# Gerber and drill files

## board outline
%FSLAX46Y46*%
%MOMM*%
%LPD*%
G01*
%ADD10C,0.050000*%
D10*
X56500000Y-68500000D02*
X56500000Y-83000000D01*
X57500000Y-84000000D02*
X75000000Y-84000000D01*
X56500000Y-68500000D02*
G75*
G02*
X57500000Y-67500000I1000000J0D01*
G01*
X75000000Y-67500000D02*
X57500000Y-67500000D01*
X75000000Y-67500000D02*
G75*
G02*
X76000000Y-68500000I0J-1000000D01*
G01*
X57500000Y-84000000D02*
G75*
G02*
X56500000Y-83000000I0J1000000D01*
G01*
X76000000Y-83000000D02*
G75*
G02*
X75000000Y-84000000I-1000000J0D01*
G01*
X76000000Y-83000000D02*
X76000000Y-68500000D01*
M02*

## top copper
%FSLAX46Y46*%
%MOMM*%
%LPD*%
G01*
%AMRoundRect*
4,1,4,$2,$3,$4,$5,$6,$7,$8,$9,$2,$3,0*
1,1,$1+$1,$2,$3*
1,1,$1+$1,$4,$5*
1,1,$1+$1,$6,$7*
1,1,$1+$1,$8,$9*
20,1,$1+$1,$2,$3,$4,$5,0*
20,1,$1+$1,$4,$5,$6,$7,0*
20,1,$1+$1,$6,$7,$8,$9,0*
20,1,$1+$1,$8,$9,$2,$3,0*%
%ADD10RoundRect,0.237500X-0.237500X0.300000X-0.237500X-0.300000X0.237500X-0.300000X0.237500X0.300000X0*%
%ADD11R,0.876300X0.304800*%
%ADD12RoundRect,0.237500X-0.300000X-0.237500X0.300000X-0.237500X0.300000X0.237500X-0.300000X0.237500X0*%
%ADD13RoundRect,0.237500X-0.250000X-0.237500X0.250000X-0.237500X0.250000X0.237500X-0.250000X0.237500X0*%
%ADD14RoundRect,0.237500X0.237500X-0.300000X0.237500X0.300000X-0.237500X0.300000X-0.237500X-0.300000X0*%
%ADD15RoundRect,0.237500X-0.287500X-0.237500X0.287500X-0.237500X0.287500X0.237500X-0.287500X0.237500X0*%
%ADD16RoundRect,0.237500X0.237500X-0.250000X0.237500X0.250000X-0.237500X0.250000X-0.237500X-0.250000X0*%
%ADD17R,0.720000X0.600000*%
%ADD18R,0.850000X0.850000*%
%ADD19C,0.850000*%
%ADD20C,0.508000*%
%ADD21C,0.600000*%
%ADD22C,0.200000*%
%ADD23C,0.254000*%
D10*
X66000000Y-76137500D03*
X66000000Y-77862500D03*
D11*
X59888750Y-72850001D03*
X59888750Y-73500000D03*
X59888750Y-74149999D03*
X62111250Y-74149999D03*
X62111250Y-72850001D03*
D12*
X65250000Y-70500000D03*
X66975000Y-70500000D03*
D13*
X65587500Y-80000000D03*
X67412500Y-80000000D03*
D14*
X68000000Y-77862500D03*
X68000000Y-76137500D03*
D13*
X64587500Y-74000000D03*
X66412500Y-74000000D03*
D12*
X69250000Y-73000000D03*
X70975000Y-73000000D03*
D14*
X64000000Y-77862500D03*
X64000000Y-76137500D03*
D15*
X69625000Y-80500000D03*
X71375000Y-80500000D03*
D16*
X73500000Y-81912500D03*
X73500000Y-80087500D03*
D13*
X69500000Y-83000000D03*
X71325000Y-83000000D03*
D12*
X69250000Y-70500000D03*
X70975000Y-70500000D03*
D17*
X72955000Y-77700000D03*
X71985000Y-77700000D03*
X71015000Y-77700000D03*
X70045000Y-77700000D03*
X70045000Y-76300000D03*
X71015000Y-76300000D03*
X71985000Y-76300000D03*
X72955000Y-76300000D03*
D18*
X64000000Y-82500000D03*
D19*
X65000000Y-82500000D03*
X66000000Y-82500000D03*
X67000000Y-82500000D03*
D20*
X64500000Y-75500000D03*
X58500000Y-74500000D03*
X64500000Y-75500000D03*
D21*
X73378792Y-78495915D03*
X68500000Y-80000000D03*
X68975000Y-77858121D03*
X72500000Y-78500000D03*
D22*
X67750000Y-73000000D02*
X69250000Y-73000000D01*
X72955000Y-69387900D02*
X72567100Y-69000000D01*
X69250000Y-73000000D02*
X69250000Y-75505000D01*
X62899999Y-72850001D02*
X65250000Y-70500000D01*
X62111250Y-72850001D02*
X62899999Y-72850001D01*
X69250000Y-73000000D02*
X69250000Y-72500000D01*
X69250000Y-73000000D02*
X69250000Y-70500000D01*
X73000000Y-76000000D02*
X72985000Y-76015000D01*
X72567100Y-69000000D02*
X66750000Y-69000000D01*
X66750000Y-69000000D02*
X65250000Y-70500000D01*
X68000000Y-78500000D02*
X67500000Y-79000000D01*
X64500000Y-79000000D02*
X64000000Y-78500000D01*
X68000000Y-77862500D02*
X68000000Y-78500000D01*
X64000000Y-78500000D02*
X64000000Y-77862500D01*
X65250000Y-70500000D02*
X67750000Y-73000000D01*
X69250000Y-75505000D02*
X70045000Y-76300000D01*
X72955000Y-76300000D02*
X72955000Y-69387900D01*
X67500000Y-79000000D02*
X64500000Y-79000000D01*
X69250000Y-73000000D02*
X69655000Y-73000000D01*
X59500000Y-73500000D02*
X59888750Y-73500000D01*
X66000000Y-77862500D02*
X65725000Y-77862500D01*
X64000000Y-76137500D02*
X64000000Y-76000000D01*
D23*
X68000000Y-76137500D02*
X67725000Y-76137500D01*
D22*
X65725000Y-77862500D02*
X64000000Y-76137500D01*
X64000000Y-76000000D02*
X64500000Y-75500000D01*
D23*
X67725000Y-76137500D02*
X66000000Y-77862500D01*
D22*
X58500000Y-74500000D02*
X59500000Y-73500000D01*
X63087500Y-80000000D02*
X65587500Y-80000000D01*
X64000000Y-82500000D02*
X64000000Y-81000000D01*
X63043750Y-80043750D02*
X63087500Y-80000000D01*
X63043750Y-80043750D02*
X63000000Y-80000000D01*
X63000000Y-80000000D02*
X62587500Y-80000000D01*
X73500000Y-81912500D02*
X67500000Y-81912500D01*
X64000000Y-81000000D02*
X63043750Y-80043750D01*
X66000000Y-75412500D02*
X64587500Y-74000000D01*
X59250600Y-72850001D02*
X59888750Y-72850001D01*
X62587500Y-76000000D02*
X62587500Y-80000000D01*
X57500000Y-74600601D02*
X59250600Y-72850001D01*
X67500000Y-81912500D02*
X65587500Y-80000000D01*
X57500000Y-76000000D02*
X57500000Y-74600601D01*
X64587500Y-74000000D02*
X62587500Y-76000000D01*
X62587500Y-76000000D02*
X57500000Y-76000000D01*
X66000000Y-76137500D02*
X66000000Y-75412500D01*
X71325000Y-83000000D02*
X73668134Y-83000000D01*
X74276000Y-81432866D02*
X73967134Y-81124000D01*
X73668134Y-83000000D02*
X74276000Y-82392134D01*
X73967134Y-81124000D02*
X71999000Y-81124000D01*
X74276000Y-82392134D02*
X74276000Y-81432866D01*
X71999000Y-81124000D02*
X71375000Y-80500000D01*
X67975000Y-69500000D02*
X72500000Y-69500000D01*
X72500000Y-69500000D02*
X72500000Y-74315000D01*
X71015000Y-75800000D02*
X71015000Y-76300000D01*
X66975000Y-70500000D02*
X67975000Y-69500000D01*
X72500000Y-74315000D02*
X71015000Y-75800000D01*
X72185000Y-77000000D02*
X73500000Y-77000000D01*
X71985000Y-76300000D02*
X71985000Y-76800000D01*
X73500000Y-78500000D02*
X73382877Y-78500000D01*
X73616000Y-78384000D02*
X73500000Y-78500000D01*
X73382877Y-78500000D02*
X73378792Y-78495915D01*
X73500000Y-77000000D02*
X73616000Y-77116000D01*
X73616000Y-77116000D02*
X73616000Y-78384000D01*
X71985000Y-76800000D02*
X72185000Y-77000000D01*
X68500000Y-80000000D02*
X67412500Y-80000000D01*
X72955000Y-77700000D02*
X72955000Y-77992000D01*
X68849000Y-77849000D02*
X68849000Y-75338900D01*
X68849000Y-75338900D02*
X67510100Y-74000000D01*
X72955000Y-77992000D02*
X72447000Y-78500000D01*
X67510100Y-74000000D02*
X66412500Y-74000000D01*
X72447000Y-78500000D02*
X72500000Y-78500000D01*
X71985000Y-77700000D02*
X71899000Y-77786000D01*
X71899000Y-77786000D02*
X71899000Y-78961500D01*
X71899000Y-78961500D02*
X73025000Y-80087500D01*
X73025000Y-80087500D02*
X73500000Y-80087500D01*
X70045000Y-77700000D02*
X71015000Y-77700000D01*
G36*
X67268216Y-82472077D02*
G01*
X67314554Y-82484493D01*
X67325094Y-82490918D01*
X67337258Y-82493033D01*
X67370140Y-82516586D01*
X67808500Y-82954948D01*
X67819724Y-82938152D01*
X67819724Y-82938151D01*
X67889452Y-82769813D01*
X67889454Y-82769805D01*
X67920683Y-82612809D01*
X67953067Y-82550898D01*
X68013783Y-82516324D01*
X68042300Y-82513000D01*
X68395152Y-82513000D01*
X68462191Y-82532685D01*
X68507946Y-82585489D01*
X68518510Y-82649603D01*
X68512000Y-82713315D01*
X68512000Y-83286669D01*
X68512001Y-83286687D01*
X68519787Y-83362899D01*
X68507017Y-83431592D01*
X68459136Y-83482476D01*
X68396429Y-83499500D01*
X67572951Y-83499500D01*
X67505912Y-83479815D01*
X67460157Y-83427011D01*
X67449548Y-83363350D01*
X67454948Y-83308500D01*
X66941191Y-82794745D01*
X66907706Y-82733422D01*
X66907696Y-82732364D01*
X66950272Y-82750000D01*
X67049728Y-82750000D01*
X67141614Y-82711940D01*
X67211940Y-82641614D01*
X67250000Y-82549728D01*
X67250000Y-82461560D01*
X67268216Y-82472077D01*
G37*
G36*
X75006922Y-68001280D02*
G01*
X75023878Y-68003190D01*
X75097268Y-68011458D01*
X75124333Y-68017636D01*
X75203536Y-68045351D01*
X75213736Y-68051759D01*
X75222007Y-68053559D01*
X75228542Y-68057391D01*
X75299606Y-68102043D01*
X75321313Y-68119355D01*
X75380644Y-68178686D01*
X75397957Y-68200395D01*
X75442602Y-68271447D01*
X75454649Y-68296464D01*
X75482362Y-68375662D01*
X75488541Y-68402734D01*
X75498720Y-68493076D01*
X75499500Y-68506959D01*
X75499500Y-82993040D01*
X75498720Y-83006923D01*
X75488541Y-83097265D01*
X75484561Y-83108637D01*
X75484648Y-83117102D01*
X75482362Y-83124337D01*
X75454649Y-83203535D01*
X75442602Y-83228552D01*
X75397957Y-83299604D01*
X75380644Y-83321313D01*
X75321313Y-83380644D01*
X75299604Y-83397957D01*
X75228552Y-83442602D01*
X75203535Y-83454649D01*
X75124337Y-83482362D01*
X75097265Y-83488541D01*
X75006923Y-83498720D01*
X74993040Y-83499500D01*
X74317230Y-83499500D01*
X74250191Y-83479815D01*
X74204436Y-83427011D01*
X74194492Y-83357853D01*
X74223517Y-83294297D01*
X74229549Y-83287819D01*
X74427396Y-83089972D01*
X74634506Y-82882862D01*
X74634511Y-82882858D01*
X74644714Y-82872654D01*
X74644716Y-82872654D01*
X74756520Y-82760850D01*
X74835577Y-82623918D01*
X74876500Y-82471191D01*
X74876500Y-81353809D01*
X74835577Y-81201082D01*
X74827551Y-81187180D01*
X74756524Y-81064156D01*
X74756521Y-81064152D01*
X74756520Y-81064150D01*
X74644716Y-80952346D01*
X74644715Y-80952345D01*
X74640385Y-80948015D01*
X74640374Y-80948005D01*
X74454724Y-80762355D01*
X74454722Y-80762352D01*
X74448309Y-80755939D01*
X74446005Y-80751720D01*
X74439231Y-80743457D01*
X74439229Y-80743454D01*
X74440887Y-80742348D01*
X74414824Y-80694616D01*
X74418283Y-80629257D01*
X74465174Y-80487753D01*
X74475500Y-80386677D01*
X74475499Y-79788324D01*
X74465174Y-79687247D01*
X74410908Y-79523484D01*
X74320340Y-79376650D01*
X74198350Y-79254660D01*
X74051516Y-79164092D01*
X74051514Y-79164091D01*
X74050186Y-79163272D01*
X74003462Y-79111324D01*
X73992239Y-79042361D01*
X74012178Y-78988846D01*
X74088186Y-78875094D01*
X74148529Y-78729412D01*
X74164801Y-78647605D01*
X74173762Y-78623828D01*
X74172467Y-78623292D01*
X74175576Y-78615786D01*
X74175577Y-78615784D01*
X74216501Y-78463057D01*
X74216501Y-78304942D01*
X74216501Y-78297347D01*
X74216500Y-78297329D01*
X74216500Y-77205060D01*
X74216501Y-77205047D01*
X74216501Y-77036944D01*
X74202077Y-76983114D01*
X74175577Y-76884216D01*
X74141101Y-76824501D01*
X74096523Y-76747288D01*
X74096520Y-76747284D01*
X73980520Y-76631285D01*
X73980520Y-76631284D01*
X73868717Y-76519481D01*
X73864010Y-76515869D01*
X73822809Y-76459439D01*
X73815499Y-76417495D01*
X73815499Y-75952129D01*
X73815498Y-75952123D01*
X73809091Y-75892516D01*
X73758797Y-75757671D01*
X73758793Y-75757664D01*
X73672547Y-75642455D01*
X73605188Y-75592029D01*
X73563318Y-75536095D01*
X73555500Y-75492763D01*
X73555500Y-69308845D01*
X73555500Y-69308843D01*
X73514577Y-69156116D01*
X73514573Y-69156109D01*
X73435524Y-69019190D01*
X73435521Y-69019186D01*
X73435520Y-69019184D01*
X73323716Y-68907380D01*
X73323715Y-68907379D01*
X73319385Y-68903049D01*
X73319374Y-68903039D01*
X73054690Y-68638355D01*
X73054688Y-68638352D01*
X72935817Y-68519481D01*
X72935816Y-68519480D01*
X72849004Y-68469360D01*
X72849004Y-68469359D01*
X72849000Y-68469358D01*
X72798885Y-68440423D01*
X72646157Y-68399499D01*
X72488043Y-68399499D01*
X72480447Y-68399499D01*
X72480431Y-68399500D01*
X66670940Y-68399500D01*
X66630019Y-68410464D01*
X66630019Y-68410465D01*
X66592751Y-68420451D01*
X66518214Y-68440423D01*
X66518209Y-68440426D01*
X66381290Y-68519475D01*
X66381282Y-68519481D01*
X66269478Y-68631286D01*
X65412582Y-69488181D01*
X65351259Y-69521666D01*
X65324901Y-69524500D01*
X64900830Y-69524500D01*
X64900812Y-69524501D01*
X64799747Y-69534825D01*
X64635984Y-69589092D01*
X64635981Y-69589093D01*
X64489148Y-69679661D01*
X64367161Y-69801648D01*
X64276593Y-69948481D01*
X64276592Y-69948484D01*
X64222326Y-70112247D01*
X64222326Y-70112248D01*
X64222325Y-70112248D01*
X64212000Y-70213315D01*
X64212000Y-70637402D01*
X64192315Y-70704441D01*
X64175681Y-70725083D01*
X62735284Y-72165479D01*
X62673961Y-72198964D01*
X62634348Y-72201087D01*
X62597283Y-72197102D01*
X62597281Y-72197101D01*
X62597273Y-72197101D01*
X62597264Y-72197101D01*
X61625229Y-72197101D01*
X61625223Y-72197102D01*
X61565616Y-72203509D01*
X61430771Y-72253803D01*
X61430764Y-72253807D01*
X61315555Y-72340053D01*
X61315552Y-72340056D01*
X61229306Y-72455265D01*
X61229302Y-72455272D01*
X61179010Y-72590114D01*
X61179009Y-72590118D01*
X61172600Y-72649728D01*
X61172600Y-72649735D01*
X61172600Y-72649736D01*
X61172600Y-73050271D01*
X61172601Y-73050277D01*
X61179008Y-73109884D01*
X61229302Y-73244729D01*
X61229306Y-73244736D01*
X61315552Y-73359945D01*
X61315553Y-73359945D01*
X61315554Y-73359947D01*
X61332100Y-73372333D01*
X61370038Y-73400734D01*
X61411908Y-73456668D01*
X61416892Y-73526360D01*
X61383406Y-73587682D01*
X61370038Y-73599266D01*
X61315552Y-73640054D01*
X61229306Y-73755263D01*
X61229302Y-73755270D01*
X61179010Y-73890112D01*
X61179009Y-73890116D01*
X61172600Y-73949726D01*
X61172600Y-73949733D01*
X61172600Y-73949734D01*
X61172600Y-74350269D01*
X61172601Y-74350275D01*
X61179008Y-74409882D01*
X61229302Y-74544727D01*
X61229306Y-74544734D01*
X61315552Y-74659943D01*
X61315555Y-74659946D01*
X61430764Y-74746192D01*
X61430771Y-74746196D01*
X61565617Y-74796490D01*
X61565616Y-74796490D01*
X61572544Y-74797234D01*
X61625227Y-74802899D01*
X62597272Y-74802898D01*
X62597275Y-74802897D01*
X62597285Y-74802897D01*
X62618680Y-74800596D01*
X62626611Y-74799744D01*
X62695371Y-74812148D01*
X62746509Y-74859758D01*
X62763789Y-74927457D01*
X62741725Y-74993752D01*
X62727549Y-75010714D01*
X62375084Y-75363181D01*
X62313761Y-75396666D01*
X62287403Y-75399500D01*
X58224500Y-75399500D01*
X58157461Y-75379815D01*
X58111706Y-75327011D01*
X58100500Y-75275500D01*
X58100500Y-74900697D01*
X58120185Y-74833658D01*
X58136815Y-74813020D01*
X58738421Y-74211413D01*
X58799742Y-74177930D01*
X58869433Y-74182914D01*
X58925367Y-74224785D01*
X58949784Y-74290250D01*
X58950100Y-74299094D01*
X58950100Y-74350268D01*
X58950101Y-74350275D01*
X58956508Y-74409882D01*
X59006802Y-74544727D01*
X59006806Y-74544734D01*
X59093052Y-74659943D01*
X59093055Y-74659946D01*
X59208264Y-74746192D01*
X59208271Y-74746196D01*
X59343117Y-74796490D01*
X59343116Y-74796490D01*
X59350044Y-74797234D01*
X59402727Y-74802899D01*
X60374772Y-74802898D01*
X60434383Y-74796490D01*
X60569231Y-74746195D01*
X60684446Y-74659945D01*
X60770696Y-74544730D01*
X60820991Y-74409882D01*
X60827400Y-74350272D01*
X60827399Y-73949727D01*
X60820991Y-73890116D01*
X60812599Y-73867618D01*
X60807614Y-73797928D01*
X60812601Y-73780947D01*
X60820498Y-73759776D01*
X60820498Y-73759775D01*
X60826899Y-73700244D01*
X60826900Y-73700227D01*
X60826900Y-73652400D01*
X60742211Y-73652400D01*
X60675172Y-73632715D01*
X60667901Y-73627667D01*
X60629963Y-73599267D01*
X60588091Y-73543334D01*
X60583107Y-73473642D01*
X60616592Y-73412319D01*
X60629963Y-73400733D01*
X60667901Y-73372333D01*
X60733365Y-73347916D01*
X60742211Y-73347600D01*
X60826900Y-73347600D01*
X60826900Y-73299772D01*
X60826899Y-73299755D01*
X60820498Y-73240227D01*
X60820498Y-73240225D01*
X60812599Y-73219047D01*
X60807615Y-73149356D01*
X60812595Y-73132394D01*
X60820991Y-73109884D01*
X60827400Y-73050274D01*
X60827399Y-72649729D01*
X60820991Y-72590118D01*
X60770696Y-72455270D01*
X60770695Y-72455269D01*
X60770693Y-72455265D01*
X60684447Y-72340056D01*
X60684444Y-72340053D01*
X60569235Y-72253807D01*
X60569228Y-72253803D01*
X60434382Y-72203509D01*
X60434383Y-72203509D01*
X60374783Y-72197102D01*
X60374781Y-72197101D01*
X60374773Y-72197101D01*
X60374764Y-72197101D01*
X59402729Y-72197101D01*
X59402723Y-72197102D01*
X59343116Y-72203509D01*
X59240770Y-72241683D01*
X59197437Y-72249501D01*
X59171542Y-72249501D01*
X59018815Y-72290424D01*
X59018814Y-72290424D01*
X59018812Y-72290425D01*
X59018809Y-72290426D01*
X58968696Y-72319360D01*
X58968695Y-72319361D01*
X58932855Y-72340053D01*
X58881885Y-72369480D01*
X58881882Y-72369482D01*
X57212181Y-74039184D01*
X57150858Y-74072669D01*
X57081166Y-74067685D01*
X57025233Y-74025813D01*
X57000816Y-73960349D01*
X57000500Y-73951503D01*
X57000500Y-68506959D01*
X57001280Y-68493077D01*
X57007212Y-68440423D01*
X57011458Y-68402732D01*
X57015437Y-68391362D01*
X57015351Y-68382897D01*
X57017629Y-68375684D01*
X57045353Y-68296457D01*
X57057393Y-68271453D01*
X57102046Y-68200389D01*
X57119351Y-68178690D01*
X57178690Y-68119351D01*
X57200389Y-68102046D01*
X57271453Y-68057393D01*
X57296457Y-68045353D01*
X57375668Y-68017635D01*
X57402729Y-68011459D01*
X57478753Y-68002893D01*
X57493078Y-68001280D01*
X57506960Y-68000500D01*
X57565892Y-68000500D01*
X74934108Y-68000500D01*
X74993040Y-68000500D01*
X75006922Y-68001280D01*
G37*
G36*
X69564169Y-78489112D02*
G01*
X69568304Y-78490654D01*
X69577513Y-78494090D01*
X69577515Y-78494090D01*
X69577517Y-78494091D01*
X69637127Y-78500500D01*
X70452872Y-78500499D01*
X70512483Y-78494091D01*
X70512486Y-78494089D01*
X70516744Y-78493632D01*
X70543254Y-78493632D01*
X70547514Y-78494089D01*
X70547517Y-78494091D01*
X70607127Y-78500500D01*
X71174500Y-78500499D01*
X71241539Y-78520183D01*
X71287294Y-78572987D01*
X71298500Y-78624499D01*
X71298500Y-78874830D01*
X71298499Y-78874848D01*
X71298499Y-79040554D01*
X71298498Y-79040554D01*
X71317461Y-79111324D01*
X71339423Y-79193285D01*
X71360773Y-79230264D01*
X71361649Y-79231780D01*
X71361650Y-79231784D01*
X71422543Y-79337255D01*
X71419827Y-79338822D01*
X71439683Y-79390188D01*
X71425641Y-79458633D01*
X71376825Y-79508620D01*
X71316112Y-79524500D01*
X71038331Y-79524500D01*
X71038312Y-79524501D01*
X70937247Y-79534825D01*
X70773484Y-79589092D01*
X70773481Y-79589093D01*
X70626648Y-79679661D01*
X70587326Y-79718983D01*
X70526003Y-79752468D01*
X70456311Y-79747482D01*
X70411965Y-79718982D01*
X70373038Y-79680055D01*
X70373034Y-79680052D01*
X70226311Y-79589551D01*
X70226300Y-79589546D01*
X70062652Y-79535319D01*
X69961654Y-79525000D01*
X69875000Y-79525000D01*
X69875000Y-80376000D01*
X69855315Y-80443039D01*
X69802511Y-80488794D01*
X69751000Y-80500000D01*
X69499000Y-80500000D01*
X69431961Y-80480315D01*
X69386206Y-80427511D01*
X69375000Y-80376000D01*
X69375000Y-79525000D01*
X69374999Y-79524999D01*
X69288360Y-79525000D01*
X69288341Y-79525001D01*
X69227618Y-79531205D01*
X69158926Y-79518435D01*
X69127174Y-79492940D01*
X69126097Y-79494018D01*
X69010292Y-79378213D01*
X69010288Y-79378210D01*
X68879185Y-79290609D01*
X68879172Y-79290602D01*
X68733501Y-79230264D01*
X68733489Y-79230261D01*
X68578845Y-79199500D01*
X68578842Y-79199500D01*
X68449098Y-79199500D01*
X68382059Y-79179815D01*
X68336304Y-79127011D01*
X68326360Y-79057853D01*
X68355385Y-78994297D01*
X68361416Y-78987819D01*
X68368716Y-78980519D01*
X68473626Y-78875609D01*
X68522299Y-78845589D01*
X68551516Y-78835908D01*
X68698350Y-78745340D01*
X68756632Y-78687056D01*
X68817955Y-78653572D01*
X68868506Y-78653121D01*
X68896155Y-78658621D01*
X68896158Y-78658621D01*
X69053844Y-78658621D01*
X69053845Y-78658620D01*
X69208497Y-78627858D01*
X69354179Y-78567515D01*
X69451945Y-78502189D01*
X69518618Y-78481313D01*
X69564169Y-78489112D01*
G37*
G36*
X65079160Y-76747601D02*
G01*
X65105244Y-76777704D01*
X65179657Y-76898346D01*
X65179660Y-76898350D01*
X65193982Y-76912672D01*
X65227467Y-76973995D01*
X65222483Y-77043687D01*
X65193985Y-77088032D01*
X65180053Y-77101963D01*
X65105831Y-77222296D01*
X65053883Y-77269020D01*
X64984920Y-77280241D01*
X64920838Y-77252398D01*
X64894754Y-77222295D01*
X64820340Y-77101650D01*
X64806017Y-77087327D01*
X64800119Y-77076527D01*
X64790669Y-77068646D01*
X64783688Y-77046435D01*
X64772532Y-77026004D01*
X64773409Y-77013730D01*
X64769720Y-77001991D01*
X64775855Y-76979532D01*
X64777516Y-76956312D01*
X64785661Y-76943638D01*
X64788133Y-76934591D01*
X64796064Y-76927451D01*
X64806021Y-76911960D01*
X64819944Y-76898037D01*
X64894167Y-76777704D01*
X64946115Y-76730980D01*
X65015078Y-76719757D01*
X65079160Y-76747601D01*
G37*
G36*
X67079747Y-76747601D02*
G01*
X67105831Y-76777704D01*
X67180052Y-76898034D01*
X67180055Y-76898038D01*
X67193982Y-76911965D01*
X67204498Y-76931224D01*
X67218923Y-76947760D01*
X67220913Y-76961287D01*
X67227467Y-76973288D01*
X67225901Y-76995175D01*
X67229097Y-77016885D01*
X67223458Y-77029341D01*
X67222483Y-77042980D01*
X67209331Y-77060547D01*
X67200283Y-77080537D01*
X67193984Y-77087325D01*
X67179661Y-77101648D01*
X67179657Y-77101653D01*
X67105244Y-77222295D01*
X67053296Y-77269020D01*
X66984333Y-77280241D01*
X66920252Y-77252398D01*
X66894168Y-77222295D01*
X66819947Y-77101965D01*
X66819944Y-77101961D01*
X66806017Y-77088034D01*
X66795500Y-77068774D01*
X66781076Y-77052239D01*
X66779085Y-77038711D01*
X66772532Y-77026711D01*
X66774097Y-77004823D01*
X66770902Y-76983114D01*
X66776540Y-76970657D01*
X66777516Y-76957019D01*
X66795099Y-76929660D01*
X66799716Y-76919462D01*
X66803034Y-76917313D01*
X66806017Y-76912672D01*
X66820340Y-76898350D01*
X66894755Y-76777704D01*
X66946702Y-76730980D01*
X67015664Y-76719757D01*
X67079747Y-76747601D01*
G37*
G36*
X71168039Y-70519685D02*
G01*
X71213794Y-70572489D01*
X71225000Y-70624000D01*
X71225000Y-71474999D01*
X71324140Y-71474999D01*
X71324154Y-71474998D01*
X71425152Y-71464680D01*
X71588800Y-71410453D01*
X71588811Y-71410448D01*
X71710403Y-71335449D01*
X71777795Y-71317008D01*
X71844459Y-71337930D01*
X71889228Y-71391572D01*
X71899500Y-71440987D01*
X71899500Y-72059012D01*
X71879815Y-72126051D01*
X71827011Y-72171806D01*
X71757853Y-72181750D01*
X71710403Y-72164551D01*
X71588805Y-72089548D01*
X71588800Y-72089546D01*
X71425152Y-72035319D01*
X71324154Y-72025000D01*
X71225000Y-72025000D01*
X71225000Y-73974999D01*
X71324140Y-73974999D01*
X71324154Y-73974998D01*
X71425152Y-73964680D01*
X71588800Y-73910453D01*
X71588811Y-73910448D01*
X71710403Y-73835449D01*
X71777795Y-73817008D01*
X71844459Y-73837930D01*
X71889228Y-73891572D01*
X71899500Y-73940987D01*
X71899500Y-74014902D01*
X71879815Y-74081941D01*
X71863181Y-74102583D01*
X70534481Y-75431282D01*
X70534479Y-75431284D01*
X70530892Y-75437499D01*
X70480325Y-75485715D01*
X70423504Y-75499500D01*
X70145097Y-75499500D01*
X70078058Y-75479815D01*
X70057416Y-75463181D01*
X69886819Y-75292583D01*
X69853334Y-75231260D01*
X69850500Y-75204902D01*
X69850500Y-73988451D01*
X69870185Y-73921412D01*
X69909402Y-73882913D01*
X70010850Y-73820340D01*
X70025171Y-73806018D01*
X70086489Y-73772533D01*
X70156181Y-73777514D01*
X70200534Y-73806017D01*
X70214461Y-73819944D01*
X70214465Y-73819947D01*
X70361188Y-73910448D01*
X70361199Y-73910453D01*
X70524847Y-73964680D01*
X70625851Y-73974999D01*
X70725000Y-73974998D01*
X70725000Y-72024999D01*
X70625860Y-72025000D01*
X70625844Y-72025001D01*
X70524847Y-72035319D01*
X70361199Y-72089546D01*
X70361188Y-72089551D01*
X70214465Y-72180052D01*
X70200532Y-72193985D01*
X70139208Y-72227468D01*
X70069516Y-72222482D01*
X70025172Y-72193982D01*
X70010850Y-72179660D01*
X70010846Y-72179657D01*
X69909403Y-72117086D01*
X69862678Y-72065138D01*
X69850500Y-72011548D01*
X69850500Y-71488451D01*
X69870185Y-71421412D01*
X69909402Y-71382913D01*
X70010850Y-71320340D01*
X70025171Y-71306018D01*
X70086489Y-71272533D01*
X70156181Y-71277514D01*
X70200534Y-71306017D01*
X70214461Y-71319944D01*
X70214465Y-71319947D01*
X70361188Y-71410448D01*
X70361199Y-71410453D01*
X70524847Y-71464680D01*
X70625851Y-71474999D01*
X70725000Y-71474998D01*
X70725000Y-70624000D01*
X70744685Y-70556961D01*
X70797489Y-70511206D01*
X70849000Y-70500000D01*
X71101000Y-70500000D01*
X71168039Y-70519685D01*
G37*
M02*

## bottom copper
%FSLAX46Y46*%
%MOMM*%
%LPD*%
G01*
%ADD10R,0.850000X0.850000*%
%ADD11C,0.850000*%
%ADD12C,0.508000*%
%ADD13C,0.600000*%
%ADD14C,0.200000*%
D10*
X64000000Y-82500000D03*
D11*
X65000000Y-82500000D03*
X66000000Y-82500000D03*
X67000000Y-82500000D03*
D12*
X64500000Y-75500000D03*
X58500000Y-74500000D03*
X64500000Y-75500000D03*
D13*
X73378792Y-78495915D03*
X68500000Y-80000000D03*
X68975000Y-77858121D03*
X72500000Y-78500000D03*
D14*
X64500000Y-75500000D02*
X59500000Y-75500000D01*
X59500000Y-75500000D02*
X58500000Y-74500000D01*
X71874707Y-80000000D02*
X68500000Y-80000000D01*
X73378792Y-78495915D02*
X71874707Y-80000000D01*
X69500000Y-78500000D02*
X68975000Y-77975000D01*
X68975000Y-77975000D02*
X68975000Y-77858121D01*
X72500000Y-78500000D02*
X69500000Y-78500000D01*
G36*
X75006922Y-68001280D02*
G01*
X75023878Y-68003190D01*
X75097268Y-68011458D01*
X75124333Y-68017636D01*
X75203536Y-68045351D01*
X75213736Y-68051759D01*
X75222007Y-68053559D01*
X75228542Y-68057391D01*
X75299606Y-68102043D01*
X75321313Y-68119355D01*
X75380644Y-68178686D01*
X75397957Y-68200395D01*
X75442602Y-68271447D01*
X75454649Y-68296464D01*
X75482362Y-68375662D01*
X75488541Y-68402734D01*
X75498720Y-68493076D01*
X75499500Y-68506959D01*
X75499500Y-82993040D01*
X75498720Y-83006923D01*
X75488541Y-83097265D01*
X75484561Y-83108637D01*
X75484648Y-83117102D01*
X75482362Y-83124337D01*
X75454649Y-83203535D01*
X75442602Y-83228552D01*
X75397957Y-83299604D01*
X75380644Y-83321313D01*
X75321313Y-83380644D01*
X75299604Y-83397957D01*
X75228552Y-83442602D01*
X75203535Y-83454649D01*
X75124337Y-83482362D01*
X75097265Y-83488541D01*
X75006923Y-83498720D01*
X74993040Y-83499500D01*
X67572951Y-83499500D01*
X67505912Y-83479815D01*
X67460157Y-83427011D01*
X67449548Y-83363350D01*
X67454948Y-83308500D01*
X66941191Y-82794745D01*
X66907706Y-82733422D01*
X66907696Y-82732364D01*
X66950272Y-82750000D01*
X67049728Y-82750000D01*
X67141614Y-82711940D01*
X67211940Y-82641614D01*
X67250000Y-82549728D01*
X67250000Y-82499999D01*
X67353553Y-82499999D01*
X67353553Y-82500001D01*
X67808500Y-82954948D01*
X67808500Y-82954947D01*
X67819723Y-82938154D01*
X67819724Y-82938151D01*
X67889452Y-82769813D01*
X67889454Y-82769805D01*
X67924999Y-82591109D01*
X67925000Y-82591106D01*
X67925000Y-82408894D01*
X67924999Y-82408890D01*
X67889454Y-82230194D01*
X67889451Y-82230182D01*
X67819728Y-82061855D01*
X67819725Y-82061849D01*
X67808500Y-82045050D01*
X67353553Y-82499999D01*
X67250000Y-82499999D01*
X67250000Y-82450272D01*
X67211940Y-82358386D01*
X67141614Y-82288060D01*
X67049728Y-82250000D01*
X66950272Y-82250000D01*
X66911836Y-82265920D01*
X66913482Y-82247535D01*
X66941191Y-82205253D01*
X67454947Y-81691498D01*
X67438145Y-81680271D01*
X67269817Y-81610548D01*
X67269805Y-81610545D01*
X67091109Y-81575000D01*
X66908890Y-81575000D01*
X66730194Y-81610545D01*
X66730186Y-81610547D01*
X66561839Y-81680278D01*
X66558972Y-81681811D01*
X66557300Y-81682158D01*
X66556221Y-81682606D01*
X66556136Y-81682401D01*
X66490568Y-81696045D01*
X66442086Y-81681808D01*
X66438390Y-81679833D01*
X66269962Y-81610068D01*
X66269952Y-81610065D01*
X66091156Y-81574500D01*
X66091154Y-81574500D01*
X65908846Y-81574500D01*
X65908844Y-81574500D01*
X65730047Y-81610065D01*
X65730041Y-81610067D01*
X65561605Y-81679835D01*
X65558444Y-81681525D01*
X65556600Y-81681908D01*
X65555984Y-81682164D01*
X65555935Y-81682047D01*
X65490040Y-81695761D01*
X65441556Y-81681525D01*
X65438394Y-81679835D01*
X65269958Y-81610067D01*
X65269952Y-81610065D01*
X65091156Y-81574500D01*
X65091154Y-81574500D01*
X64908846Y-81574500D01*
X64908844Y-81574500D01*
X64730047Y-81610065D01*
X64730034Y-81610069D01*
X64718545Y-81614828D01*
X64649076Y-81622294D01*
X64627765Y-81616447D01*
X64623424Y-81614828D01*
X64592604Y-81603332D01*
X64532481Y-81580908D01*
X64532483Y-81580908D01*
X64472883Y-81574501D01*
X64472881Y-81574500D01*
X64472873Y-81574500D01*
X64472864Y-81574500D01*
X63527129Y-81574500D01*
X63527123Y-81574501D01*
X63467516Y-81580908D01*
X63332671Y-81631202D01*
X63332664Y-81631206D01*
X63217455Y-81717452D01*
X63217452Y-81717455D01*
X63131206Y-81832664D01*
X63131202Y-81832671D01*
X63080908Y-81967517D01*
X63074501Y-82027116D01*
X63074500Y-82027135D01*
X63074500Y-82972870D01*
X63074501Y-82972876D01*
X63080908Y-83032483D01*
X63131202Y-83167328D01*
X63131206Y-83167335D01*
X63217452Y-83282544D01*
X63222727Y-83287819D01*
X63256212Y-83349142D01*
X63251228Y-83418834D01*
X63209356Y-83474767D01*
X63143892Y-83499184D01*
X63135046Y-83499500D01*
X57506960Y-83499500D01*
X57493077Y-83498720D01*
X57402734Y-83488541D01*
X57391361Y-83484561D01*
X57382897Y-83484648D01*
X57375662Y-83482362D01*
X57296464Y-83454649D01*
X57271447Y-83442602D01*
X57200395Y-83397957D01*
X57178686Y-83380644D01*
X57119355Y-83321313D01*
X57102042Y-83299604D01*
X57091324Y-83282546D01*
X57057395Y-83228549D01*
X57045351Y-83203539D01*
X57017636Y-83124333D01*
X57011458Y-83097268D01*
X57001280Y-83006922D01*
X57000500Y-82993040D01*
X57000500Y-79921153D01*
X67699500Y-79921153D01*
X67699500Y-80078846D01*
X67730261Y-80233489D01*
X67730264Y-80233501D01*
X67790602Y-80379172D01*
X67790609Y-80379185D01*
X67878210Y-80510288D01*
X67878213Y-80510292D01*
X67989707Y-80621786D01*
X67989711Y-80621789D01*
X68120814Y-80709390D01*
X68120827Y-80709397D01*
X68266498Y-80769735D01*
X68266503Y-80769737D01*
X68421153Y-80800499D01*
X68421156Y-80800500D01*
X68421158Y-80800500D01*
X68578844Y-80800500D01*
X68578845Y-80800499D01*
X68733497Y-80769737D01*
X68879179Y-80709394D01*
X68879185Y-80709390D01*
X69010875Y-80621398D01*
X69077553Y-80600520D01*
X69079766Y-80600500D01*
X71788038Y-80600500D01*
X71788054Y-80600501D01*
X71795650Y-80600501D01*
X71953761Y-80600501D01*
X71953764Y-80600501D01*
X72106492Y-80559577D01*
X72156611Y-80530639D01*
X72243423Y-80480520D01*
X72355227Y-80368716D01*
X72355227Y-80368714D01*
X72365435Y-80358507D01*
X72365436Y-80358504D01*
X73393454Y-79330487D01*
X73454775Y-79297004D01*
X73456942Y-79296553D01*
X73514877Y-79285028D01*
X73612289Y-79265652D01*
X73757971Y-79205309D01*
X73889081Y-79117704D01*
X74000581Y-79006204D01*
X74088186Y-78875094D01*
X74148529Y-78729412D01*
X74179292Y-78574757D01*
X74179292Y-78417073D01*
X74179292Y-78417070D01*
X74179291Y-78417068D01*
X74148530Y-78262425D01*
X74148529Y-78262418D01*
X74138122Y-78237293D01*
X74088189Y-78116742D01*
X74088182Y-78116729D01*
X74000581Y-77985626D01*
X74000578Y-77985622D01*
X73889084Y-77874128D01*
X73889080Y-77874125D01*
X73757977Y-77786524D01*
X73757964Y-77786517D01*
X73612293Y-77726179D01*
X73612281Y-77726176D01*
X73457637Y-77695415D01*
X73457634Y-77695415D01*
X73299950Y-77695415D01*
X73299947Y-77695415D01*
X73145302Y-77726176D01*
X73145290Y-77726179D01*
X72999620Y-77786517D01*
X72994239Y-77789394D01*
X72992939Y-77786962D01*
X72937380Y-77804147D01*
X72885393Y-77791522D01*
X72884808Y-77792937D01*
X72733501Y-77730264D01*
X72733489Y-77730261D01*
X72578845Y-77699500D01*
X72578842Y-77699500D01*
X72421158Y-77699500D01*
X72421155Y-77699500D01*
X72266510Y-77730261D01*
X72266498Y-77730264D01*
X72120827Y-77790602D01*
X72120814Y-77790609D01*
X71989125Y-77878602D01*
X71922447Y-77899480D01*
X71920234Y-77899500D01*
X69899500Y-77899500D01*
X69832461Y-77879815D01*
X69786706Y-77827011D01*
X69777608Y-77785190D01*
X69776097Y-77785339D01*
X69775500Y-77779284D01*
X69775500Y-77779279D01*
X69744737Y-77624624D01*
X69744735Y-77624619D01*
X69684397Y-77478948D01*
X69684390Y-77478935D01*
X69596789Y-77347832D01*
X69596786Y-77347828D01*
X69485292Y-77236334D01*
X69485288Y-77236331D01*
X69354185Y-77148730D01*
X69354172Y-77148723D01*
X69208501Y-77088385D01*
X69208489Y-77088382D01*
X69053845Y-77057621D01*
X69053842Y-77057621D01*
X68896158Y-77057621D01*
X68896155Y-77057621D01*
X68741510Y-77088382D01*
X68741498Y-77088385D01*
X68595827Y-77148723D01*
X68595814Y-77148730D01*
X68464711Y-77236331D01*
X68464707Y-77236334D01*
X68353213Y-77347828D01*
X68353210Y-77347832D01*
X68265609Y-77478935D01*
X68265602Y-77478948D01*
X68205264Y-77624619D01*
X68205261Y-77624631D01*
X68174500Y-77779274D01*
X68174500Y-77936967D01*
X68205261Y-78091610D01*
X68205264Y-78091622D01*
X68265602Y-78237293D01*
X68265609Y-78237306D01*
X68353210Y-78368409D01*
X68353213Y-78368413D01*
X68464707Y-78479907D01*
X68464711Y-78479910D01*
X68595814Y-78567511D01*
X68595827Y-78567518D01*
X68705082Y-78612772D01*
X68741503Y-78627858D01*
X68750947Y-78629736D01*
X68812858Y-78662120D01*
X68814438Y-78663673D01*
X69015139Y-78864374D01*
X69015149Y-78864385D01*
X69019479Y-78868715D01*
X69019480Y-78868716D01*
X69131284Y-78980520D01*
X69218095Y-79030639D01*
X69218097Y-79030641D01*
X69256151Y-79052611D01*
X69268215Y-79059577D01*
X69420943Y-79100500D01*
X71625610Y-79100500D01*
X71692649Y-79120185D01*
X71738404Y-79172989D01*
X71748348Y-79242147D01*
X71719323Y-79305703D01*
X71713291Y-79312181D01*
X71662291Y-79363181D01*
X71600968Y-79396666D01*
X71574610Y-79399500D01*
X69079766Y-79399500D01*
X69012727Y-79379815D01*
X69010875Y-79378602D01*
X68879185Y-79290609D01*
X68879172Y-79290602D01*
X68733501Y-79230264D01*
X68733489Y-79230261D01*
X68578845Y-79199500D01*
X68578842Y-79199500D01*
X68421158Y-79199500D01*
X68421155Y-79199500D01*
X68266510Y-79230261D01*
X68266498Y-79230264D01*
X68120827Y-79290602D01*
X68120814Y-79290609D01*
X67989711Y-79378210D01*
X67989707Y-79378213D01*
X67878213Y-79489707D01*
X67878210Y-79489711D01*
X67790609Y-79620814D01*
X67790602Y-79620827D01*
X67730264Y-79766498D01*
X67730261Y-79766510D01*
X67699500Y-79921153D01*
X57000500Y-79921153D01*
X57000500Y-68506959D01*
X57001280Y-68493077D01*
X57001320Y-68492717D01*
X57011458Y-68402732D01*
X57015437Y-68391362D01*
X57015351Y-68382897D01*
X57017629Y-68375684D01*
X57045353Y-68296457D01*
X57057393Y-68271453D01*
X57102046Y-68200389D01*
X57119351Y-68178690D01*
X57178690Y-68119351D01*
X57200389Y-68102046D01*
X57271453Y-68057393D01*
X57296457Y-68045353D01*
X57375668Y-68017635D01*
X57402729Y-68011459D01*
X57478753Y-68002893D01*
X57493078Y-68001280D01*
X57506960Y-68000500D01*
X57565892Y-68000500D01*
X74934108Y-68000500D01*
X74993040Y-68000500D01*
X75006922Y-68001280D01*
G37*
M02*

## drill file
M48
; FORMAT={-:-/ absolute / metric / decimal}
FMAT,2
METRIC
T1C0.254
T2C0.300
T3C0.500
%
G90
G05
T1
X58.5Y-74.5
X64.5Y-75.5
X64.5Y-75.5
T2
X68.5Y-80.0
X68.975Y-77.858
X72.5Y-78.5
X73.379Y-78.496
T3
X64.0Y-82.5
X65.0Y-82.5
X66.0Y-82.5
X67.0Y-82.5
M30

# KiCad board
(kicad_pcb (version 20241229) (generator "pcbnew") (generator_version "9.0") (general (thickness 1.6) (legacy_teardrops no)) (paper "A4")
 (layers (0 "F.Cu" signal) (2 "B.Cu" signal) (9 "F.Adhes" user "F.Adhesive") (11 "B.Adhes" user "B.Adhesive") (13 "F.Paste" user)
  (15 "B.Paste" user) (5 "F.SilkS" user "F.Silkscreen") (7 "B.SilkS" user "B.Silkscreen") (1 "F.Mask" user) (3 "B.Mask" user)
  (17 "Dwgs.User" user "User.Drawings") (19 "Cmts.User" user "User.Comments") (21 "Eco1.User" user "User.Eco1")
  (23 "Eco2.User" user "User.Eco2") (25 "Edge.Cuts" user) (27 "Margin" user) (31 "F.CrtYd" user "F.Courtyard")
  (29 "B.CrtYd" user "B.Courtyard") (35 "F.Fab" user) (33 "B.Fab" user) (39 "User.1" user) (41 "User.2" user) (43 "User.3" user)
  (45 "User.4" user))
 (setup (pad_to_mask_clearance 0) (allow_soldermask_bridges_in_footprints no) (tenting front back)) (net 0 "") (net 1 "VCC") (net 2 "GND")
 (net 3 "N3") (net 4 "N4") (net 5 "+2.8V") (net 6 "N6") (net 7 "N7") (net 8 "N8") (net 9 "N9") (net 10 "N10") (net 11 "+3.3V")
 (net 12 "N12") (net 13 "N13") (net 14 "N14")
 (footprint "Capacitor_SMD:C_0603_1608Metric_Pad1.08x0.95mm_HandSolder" (layer "F.Cu") (at 66 77 -90)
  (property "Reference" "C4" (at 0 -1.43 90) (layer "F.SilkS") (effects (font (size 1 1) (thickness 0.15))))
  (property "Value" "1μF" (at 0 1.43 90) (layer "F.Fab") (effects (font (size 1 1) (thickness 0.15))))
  (pad "1" smd roundrect (at -0.8625 0 270) (size 1.075 0.95) (layers "F.Cu" "F.Mask" "F.Paste") (roundrect_rratio 0.25) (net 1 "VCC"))
  (pad "2" smd roundrect (at 0.8625 0 270) (size 1.075 0.95) (layers "F.Cu" "F.Mask" "F.Paste") (roundrect_rratio 0.25) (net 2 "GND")))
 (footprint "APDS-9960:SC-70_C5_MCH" (layer "F.Cu") (at 61 73.5)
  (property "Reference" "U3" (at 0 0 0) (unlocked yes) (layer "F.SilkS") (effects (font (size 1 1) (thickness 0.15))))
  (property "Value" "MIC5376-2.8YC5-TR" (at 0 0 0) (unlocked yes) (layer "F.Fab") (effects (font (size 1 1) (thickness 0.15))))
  (pad "1" smd rect (at -1.11125 -0.649999) (size 0.8763 0.3048) (layers "F.Cu" "F.Mask" "F.Paste") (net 1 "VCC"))
  (pad "2" smd rect (at -1.11125 0) (size 0.8763 0.3048) (layers "F.Cu" "F.Mask" "F.Paste") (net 2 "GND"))
  (pad "3" smd rect (at -1.11125 0.649999) (size 0.8763 0.3048) (layers "F.Cu" "F.Mask" "F.Paste") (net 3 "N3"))
  (pad "4" smd rect (at 1.11125 0.649999) (size 0.8763 0.3048) (layers "F.Cu" "F.Mask" "F.Paste") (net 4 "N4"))
  (pad "5" smd rect (at 1.11125 -0.649999) (size 0.8763 0.3048) (layers "F.Cu" "F.Mask" "F.Paste") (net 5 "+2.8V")))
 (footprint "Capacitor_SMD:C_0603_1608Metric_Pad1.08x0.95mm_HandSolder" (layer "F.Cu") (at 66.1125 70.5)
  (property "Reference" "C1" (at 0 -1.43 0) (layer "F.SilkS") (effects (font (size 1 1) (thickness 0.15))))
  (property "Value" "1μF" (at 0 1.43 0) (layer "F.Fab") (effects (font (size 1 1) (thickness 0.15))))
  (pad "1" smd roundrect (at -0.8625 0) (size 1.075 0.95) (layers "F.Cu" "F.Mask" "F.Paste") (roundrect_rratio 0.25) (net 5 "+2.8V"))
  (pad "2" smd roundrect (at 0.8625 0) (size 1.075 0.95) (layers "F.Cu" "F.Mask" "F.Paste") (roundrect_rratio 0.25) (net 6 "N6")))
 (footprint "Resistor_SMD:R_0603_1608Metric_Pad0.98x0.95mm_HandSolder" (layer "F.Cu") (at 66.5 80)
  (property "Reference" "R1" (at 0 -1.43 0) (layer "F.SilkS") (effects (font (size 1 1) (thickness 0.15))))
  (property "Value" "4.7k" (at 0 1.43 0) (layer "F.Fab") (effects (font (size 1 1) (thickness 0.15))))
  (pad "1" smd roundrect (at -0.9125 0) (size 0.975 0.95) (layers "F.Cu" "F.Mask" "F.Paste") (roundrect_rratio 0.25) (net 1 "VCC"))
  (pad "2" smd roundrect (at 0.9125 0) (size 0.975 0.95) (layers "F.Cu" "F.Mask" "F.Paste") (roundrect_rratio 0.25) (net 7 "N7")))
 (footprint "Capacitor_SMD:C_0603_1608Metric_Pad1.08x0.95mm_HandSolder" (layer "F.Cu") (at 68 77 90)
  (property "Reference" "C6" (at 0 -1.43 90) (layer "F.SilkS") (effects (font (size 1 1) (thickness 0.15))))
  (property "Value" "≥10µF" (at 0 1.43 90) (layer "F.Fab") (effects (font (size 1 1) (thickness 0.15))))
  (pad "1" smd roundrect (at -0.8625 0 90) (size 1.075 0.95) (layers "F.Cu" "F.Mask" "F.Paste") (roundrect_rratio 0.25) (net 5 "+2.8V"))
  (pad "2" smd roundrect (at 0.8625 0 90) (size 1.075 0.95) (layers "F.Cu" "F.Mask" "F.Paste") (roundrect_rratio 0.25) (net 2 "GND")))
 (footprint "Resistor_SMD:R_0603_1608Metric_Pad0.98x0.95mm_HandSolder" (layer "F.Cu") (at 65.5 74)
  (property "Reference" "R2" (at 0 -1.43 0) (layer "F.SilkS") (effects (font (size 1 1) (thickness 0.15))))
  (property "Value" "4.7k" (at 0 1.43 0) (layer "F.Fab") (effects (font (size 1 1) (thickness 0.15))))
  (pad "1" smd roundrect (at -0.9125 0) (size 0.975 0.95) (layers "F.Cu" "F.Mask" "F.Paste") (roundrect_rratio 0.25) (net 1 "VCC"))
  (pad "2" smd roundrect (at 0.9125 0) (size 0.975 0.95) (layers "F.Cu" "F.Mask" "F.Paste") (roundrect_rratio 0.25) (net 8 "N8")))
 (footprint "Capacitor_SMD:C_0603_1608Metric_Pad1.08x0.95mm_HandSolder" (layer "F.Cu") (at 70.1125 73)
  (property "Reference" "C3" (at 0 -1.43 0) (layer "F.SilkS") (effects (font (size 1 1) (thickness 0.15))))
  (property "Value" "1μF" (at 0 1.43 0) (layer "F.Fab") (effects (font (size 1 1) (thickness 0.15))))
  (pad "1" smd roundrect (at -0.8625 0) (size 1.075 0.95) (layers "F.Cu" "F.Mask" "F.Paste") (roundrect_rratio 0.25) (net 5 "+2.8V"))
  (pad "2" smd roundrect (at 0.8625 0) (size 1.075 0.95) (layers "F.Cu" "F.Mask" "F.Paste") (roundrect_rratio 0.25) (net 2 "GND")))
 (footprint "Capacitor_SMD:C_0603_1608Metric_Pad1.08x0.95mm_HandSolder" (layer "F.Cu") (at 64 77 90)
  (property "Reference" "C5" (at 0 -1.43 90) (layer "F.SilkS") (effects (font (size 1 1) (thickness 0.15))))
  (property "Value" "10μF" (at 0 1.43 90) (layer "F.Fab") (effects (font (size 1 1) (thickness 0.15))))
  (pad "1" smd roundrect (at -0.8625 0 90) (size 1.075 0.95) (layers "F.Cu" "F.Mask" "F.Paste") (roundrect_rratio 0.25) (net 5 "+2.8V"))
  (pad "2" smd roundrect (at 0.8625 0 90) (size 1.075 0.95) (layers "F.Cu" "F.Mask" "F.Paste") (roundrect_rratio 0.25) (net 2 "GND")))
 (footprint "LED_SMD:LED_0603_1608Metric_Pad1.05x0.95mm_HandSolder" (layer "F.Cu") (at 70.5 80.5)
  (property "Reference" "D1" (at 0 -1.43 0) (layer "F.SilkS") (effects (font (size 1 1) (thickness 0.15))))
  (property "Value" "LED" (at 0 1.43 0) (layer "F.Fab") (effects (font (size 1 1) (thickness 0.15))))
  (pad "1" smd roundrect (at -0.875 0) (size 1.05 0.95) (layers "F.Cu" "F.Mask" "F.Paste") (roundrect_rratio 0.25) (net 2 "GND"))
  (pad "2" smd roundrect (at 0.875 0) (size 1.05 0.95) (layers "F.Cu" "F.Mask" "F.Paste") (roundrect_rratio 0.25) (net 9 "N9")))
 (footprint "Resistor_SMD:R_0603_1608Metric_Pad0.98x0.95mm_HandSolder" (layer "F.Cu") (at 73.5 81 90)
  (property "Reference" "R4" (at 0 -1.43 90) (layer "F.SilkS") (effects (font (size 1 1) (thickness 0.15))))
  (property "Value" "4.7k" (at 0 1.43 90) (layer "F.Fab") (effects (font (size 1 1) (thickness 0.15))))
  (pad "1" smd roundrect (at -0.9125 0 90) (size 0.975 0.95) (layers "F.Cu" "F.Mask" "F.Paste") (roundrect_rratio 0.25) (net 1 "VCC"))
  (pad "2" smd roundrect (at 0.9125 0 90) (size 0.975 0.95) (layers "F.Cu" "F.Mask" "F.Paste") (roundrect_rratio 0.25) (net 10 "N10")))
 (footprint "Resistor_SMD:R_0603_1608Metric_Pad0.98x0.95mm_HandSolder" (layer "F.Cu") (at 70.4125 83)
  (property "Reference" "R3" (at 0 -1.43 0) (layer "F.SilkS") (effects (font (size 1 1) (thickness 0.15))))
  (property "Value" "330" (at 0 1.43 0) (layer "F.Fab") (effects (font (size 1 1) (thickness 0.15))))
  (pad "1" smd roundrect (at -0.9125 0) (size 0.975 0.95) (layers "F.Cu" "F.Mask" "F.Paste") (roundrect_rratio 0.25) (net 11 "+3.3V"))
  (pad "2" smd roundrect (at 0.9125 0) (size 0.975 0.95) (layers "F.Cu" "F.Mask" "F.Paste") (roundrect_rratio 0.25) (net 9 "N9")))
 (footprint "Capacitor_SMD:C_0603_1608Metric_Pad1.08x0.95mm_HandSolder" (layer "F.Cu") (at 70.1125 70.5)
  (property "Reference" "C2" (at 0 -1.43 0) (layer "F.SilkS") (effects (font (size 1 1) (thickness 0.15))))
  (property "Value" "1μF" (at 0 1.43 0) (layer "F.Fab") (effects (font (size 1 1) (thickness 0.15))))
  (pad "1" smd roundrect (at -0.8625 0) (size 1.075 0.95) (layers "F.Cu" "F.Mask" "F.Paste") (roundrect_rratio 0.25) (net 5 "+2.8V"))
  (pad "2" smd roundrect (at 0.8625 0) (size 1.075 0.95) (layers "F.Cu" "F.Mask" "F.Paste") (roundrect_rratio 0.25) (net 2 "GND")))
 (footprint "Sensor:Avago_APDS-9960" (layer "F.Cu") (at 71.5 77 180)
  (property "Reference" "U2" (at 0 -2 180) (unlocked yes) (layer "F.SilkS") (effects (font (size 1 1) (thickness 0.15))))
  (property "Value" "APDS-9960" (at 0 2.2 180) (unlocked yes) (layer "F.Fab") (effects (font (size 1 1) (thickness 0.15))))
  (pad "1" smd rect (at -1.455 -0.7 180) (size 0.72 0.6) (layers "F.Cu" "F.Mask" "F.Paste") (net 8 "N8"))
  (pad "2" smd rect (at -0.485 -0.7 180) (size 0.72 0.6) (layers "F.Cu" "F.Mask" "F.Paste") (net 10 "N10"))
  (pad "3" smd rect (at 0.485 -0.7 180) (size 0.72 0.6) (layers "F.Cu" "F.Mask" "F.Paste") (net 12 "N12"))
  (pad "4" smd rect (at 1.455 -0.7 180) (size 0.72 0.6) (layers "F.Cu" "F.Mask" "F.Paste") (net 12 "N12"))
  (pad "5" smd rect (at 1.455 0.7 180) (size 0.72 0.6) (layers "F.Cu" "F.Mask" "F.Paste") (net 5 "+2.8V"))
  (pad "6" smd rect (at 0.485 0.7 180) (size 0.72 0.6) (layers "F.Cu" "F.Mask" "F.Paste") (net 6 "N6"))
  (pad "7" smd rect (at -0.485 0.7 180) (size 0.72 0.6) (layers "F.Cu" "F.Mask" "F.Paste") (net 7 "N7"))
  (pad "8" smd rect (at -1.455 0.7 180) (size 0.72 0.6) (layers "F.Cu" "F.Mask" "F.Paste") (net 5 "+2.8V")))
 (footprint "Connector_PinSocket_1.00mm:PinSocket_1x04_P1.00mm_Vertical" (layer "F.Cu") (at 64 82.5 90)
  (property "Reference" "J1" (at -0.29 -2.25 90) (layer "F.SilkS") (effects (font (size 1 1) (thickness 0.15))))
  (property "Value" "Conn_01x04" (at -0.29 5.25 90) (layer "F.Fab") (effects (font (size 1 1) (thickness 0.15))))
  (pad "1" thru_hole rect (at 0 0 90) (size 0.85 0.85) (drill 0.5) (layers "*.Cu" "*.Mask") (remove_unused_layers no) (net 1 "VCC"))
  (pad "2" thru_hole circle (at 0 1 90) (size 0.85 0.85) (drill 0.5) (layers "*.Cu" "*.Mask") (remove_unused_layers no) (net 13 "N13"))
  (pad "3" thru_hole circle (at 0 2 90) (size 0.85 0.85) (drill 0.5) (layers "*.Cu" "*.Mask") (remove_unused_layers no) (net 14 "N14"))
  (pad "4" thru_hole circle (at 0 3 90) (size 0.85 0.85) (drill 0.5) (layers "*.Cu" "*.Mask") (remove_unused_layers no) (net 2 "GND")))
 (gr_line (start 56.5 68.5) (end 56.5 83) (stroke (width 0.05) (type default)) (layer "Edge.Cuts"))
 (gr_line (start 57.5 84) (end 75 84) (stroke (width 0.05) (type default)) (layer "Edge.Cuts"))
 (gr_arc (start 56.5 68.5) (mid 56.792893 67.792893) (end 57.5 67.5) (stroke (width 0.05) (type default)) (layer "Edge.Cuts"))
 (gr_line (start 75 67.5) (end 57.5 67.5) (stroke (width 0.05) (type default)) (layer "Edge.Cuts"))
 (gr_arc (start 75 67.5) (mid 75.707107 67.792893) (end 76 68.5) (stroke (width 0.05) (type default)) (layer "Edge.Cuts"))
 (gr_arc (start 57.5 84) (mid 56.792893 83.707107) (end 56.5 83) (stroke (width 0.05) (type default)) (layer "Edge.Cuts"))
 (gr_arc (start 76 83) (mid 75.707107 83.707107) (end 75 84) (stroke (width 0.05) (type default)) (layer "Edge.Cuts"))
 (gr_line (start 76 83) (end 76 68.5) (stroke (width 0.05) (type default)) (layer "Edge.Cuts"))
 (segment (start 67.75 73) (end 69.25 73) (width 0.2) (layer "F.Cu") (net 5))
 (segment (start 72.955 69.3879) (end 72.5671 69) (width 0.2) (layer "F.Cu") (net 5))
 (segment (start 69.25 73) (end 69.25 75.505) (width 0.2) (layer "F.Cu") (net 5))
 (segment (start 62.899999 72.850001) (end 65.25 70.5) (width 0.2) (layer "F.Cu") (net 5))
 (segment (start 62.11125 72.850001) (end 62.899999 72.850001) (width 0.2) (layer "F.Cu") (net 5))
 (segment (start 69.25 73) (end 69.25 72.5) (width 0.2) (layer "F.Cu") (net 5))
 (segment (start 69.25 73) (end 69.25 70.5) (width 0.2) (layer "F.Cu") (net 5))
 (segment (start 73 76) (end 72.985 76.015) (width 0.2) (layer "F.Cu") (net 5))
 (segment (start 72.5671 69) (end 66.75 69) (width 0.2) (layer "F.Cu") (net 5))
 (segment (start 66.75 69) (end 65.25 70.5) (width 0.2) (layer "F.Cu") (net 5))
 (segment (start 68 78.5) (end 67.5 79) (width 0.2) (layer "F.Cu") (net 5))
 (segment (start 64.5 79) (end 64 78.5) (width 0.2) (layer "F.Cu") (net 5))
 (segment (start 68 77.8625) (end 68 78.5) (width 0.2) (layer "F.Cu") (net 5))
 (segment (start 64 78.5) (end 64 77.8625) (width 0.2) (layer "F.Cu") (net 5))
 (segment (start 65.25 70.5) (end 67.75 73) (width 0.2) (layer "F.Cu") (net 5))
 (segment (start 69.25 75.505) (end 70.045 76.3) (width 0.2) (layer "F.Cu") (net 5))
 (segment (start 72.955 76.3) (end 72.955 69.3879) (width 0.2) (layer "F.Cu") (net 5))
 (segment (start 67.5 79) (end 64.5 79) (width 0.2) (layer "F.Cu") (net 5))
 (segment (start 69.25 73) (end 69.655 73) (width 0.2) (layer "F.Cu") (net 5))
 (segment (start 59.5 73.5) (end 59.88875 73.5) (width 0.2) (layer "F.Cu") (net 2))
 (segment (start 66 77.8625) (end 65.725 77.8625) (width 0.2) (layer "F.Cu") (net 2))
 (segment (start 64 76.1375) (end 64 76) (width 0.2) (layer "F.Cu") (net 2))
 (segment (start 68 76.1375) (end 67.725 76.1375) (width 0.254) (layer "F.Cu") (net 2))
 (segment (start 65.725 77.8625) (end 64 76.1375) (width 0.2) (layer "F.Cu") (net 2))
 (segment (start 64 76) (end 64.5 75.5) (width 0.2) (layer "F.Cu") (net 2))
 (segment (start 67.725 76.1375) (end 66 77.8625) (width 0.254) (layer "F.Cu") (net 2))
 (segment (start 58.5 74.5) (end 59.5 73.5) (width 0.2) (layer "F.Cu") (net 2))
 (via (at 64.5 75.5) (size 0.508) (drill 0.254) (layers "F.Cu" "B.Cu") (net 2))
 (via (at 58.5 74.5) (size 0.508) (drill 0.254) (layers "F.Cu" "B.Cu") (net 2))
 (via (at 64.5 75.5) (size 0.508) (drill 0.254) (layers "F.Cu" "B.Cu") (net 2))
 (segment (start 64.5 75.5) (end 59.5 75.5) (width 0.2) (layer "B.Cu") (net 2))
 (segment (start 59.5 75.5) (end 58.5 74.5) (width 0.2) (layer "B.Cu") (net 2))
 (segment (start 63.0875 80) (end 65.5875 80) (width 0.2) (layer "F.Cu") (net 1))
 (segment (start 64 82.5) (end 64 81) (width 0.2) (layer "F.Cu") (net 1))
 (segment (start 63.04375 80.04375) (end 63.0875 80) (width 0.2) (layer "F.Cu") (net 1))
 (segment (start 63.04375 80.04375) (end 63 80) (width 0.2) (layer "F.Cu") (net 1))
 (segment (start 63 80) (end 62.5875 80) (width 0.2) (layer "F.Cu") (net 1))
 (segment (start 73.5 81.9125) (end 67.5 81.9125) (width 0.2) (layer "F.Cu") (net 1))
 (segment (start 64 81) (end 63.04375 80.04375) (width 0.2) (layer "F.Cu") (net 1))
 (segment (start 66 75.4125) (end 64.5875 74) (width 0.2) (layer "F.Cu") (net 1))
 (segment (start 59.2506 72.850001) (end 59.88875 72.850001) (width 0.2) (layer "F.Cu") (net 1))
 (segment (start 62.5875 76) (end 62.5875 80) (width 0.2) (layer "F.Cu") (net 1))
 (segment (start 57.5 74.600601) (end 59.2506 72.850001) (width 0.2) (layer "F.Cu") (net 1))
 (segment (start 67.5 81.9125) (end 65.5875 80) (width 0.2) (layer "F.Cu") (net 1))
 (segment (start 57.5 76) (end 57.5 74.600601) (width 0.2) (layer "F.Cu") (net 1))
 (segment (start 64.5875 74) (end 62.5875 76) (width 0.2) (layer "F.Cu") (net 1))
 (segment (start 62.5875 76) (end 57.5 76) (width 0.2) (layer "F.Cu") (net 1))
 (segment (start 66 76.1375) (end 66 75.4125) (width 0.2) (layer "F.Cu") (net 1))
 (segment (start 71.325 83) (end 73.668134 83) (width 0.2) (layer "F.Cu") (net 9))
 (segment (start 74.276 81.432866) (end 73.967134 81.124) (width 0.2) (layer "F.Cu") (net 9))
 (segment (start 73.668134 83) (end 74.276 82.392134) (width 0.2) (layer "F.Cu") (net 9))
 (segment (start 73.967134 81.124) (end 71.999 81.124) (width 0.2) (layer "F.Cu") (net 9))
 (segment (start 74.276 82.392134) (end 74.276 81.432866) (width 0.2) (layer "F.Cu") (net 9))
 (segment (start 71.999 81.124) (end 71.375 80.5) (width 0.2) (layer "F.Cu") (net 9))
 (segment (start 67.975 69.5) (end 72.5 69.5) (width 0.2) (layer "F.Cu") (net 6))
 (segment (start 72.5 69.5) (end 72.5 74.315) (width 0.2) (layer "F.Cu") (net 6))
 (segment (start 71.015 75.8) (end 71.015 76.3) (width 0.2) (layer "F.Cu") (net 6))
 (segment (start 66.975 70.5) (end 67.975 69.5) (width 0.2) (layer "F.Cu") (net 6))
 (segment (start 72.5 74.315) (end 71.015 75.8) (width 0.2) (layer "F.Cu") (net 6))
 (segment (start 72.185 77) (end 73.5 77) (width 0.2) (layer "F.Cu") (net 7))
 (segment (start 71.985 76.3) (end 71.985 76.8) (width 0.2) (layer "F.Cu") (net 7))
 (segment (start 73.5 78.5) (end 73.382877 78.5) (width 0.2) (layer "F.Cu") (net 7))
 (segment (start 73.616 78.384) (end 73.5 78.5) (width 0.2) (layer "F.Cu") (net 7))
 (segment (start 73.382877 78.5) (end 73.378792 78.495915) (width 0.2) (layer "F.Cu") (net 7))
 (segment (start 73.5 77) (end 73.616 77.116) (width 0.2) (layer "F.Cu") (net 7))
 (segment (start 73.616 77.116) (end 73.616 78.384) (width 0.2) (layer "F.Cu") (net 7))
 (segment (start 71.985 76.8) (end 72.185 77) (width 0.2) (layer "F.Cu") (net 7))
 (segment (start 68.5 80) (end 67.4125 80) (width 0.2) (layer "F.Cu") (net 7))
 (via (at 73.378792 78.495915) (size 0.6) (drill 0.3) (layers "F.Cu" "B.Cu") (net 7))
 (via (at 68.5 80) (size 0.6) (drill 0.3) (layers "F.Cu" "B.Cu") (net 7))
 (segment (start 71.874707 80) (end 68.5 80) (width 0.2) (layer "B.Cu") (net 7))
 (segment (start 73.378792 78.495915) (end 71.874707 80) (width 0.2) (layer "B.Cu") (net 7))
 (segment (start 72.955 77.7) (end 72.955 77.992) (width 0.2) (layer "F.Cu") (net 8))
 (segment (start 68.849 77.849) (end 68.849 75.3389) (width 0.2) (layer "F.Cu") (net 8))
 (segment (start 68.849 75.3389) (end 67.5101 74) (width 0.2) (layer "F.Cu") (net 8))
 (segment (start 72.955 77.992) (end 72.447 78.5) (width 0.2) (layer "F.Cu") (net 8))
 (segment (start 67.5101 74) (end 66.4125 74) (width 0.2) (layer "F.Cu") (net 8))
 (segment (start 72.447 78.5) (end 72.5 78.5) (width 0.2) (layer "F.Cu") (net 8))
 (via (at 68.975 77.858121) (size 0.6) (drill 0.3) (layers "F.Cu" "B.Cu") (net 8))
 (via (at 72.5 78.5) (size 0.6) (drill 0.3) (layers "F.Cu" "B.Cu") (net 8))
 (segment (start 69.5 78.5) (end 68.975 77.975) (width 0.2) (layer "B.Cu") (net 8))
 (segment (start 68.975 77.975) (end 68.975 77.858121) (width 0.2) (layer "B.Cu") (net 8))
 (segment (start 72.5 78.5) (end 69.5 78.5) (width 0.2) (layer "B.Cu") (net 8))
 (segment (start 71.985 77.7) (end 71.899 77.786) (width 0.2) (layer "F.Cu") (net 10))
 (segment (start 71.899 77.786) (end 71.899 78.9615) (width 0.2) (layer "F.Cu") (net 10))
 (segment (start 71.899 78.9615) (end 73.025 80.0875) (width 0.2) (layer "F.Cu") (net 10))
 (segment (start 73.025 80.0875) (end 73.5 80.0875) (width 0.2) (layer "F.Cu") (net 10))
 (segment (start 70.045 77.7) (end 71.015 77.7) (width 0.2) (layer "F.Cu") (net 12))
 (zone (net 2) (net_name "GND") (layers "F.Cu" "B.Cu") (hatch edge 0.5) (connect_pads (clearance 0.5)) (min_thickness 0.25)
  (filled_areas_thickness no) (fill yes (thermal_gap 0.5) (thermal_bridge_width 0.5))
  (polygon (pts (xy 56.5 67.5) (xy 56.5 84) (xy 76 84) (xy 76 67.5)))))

